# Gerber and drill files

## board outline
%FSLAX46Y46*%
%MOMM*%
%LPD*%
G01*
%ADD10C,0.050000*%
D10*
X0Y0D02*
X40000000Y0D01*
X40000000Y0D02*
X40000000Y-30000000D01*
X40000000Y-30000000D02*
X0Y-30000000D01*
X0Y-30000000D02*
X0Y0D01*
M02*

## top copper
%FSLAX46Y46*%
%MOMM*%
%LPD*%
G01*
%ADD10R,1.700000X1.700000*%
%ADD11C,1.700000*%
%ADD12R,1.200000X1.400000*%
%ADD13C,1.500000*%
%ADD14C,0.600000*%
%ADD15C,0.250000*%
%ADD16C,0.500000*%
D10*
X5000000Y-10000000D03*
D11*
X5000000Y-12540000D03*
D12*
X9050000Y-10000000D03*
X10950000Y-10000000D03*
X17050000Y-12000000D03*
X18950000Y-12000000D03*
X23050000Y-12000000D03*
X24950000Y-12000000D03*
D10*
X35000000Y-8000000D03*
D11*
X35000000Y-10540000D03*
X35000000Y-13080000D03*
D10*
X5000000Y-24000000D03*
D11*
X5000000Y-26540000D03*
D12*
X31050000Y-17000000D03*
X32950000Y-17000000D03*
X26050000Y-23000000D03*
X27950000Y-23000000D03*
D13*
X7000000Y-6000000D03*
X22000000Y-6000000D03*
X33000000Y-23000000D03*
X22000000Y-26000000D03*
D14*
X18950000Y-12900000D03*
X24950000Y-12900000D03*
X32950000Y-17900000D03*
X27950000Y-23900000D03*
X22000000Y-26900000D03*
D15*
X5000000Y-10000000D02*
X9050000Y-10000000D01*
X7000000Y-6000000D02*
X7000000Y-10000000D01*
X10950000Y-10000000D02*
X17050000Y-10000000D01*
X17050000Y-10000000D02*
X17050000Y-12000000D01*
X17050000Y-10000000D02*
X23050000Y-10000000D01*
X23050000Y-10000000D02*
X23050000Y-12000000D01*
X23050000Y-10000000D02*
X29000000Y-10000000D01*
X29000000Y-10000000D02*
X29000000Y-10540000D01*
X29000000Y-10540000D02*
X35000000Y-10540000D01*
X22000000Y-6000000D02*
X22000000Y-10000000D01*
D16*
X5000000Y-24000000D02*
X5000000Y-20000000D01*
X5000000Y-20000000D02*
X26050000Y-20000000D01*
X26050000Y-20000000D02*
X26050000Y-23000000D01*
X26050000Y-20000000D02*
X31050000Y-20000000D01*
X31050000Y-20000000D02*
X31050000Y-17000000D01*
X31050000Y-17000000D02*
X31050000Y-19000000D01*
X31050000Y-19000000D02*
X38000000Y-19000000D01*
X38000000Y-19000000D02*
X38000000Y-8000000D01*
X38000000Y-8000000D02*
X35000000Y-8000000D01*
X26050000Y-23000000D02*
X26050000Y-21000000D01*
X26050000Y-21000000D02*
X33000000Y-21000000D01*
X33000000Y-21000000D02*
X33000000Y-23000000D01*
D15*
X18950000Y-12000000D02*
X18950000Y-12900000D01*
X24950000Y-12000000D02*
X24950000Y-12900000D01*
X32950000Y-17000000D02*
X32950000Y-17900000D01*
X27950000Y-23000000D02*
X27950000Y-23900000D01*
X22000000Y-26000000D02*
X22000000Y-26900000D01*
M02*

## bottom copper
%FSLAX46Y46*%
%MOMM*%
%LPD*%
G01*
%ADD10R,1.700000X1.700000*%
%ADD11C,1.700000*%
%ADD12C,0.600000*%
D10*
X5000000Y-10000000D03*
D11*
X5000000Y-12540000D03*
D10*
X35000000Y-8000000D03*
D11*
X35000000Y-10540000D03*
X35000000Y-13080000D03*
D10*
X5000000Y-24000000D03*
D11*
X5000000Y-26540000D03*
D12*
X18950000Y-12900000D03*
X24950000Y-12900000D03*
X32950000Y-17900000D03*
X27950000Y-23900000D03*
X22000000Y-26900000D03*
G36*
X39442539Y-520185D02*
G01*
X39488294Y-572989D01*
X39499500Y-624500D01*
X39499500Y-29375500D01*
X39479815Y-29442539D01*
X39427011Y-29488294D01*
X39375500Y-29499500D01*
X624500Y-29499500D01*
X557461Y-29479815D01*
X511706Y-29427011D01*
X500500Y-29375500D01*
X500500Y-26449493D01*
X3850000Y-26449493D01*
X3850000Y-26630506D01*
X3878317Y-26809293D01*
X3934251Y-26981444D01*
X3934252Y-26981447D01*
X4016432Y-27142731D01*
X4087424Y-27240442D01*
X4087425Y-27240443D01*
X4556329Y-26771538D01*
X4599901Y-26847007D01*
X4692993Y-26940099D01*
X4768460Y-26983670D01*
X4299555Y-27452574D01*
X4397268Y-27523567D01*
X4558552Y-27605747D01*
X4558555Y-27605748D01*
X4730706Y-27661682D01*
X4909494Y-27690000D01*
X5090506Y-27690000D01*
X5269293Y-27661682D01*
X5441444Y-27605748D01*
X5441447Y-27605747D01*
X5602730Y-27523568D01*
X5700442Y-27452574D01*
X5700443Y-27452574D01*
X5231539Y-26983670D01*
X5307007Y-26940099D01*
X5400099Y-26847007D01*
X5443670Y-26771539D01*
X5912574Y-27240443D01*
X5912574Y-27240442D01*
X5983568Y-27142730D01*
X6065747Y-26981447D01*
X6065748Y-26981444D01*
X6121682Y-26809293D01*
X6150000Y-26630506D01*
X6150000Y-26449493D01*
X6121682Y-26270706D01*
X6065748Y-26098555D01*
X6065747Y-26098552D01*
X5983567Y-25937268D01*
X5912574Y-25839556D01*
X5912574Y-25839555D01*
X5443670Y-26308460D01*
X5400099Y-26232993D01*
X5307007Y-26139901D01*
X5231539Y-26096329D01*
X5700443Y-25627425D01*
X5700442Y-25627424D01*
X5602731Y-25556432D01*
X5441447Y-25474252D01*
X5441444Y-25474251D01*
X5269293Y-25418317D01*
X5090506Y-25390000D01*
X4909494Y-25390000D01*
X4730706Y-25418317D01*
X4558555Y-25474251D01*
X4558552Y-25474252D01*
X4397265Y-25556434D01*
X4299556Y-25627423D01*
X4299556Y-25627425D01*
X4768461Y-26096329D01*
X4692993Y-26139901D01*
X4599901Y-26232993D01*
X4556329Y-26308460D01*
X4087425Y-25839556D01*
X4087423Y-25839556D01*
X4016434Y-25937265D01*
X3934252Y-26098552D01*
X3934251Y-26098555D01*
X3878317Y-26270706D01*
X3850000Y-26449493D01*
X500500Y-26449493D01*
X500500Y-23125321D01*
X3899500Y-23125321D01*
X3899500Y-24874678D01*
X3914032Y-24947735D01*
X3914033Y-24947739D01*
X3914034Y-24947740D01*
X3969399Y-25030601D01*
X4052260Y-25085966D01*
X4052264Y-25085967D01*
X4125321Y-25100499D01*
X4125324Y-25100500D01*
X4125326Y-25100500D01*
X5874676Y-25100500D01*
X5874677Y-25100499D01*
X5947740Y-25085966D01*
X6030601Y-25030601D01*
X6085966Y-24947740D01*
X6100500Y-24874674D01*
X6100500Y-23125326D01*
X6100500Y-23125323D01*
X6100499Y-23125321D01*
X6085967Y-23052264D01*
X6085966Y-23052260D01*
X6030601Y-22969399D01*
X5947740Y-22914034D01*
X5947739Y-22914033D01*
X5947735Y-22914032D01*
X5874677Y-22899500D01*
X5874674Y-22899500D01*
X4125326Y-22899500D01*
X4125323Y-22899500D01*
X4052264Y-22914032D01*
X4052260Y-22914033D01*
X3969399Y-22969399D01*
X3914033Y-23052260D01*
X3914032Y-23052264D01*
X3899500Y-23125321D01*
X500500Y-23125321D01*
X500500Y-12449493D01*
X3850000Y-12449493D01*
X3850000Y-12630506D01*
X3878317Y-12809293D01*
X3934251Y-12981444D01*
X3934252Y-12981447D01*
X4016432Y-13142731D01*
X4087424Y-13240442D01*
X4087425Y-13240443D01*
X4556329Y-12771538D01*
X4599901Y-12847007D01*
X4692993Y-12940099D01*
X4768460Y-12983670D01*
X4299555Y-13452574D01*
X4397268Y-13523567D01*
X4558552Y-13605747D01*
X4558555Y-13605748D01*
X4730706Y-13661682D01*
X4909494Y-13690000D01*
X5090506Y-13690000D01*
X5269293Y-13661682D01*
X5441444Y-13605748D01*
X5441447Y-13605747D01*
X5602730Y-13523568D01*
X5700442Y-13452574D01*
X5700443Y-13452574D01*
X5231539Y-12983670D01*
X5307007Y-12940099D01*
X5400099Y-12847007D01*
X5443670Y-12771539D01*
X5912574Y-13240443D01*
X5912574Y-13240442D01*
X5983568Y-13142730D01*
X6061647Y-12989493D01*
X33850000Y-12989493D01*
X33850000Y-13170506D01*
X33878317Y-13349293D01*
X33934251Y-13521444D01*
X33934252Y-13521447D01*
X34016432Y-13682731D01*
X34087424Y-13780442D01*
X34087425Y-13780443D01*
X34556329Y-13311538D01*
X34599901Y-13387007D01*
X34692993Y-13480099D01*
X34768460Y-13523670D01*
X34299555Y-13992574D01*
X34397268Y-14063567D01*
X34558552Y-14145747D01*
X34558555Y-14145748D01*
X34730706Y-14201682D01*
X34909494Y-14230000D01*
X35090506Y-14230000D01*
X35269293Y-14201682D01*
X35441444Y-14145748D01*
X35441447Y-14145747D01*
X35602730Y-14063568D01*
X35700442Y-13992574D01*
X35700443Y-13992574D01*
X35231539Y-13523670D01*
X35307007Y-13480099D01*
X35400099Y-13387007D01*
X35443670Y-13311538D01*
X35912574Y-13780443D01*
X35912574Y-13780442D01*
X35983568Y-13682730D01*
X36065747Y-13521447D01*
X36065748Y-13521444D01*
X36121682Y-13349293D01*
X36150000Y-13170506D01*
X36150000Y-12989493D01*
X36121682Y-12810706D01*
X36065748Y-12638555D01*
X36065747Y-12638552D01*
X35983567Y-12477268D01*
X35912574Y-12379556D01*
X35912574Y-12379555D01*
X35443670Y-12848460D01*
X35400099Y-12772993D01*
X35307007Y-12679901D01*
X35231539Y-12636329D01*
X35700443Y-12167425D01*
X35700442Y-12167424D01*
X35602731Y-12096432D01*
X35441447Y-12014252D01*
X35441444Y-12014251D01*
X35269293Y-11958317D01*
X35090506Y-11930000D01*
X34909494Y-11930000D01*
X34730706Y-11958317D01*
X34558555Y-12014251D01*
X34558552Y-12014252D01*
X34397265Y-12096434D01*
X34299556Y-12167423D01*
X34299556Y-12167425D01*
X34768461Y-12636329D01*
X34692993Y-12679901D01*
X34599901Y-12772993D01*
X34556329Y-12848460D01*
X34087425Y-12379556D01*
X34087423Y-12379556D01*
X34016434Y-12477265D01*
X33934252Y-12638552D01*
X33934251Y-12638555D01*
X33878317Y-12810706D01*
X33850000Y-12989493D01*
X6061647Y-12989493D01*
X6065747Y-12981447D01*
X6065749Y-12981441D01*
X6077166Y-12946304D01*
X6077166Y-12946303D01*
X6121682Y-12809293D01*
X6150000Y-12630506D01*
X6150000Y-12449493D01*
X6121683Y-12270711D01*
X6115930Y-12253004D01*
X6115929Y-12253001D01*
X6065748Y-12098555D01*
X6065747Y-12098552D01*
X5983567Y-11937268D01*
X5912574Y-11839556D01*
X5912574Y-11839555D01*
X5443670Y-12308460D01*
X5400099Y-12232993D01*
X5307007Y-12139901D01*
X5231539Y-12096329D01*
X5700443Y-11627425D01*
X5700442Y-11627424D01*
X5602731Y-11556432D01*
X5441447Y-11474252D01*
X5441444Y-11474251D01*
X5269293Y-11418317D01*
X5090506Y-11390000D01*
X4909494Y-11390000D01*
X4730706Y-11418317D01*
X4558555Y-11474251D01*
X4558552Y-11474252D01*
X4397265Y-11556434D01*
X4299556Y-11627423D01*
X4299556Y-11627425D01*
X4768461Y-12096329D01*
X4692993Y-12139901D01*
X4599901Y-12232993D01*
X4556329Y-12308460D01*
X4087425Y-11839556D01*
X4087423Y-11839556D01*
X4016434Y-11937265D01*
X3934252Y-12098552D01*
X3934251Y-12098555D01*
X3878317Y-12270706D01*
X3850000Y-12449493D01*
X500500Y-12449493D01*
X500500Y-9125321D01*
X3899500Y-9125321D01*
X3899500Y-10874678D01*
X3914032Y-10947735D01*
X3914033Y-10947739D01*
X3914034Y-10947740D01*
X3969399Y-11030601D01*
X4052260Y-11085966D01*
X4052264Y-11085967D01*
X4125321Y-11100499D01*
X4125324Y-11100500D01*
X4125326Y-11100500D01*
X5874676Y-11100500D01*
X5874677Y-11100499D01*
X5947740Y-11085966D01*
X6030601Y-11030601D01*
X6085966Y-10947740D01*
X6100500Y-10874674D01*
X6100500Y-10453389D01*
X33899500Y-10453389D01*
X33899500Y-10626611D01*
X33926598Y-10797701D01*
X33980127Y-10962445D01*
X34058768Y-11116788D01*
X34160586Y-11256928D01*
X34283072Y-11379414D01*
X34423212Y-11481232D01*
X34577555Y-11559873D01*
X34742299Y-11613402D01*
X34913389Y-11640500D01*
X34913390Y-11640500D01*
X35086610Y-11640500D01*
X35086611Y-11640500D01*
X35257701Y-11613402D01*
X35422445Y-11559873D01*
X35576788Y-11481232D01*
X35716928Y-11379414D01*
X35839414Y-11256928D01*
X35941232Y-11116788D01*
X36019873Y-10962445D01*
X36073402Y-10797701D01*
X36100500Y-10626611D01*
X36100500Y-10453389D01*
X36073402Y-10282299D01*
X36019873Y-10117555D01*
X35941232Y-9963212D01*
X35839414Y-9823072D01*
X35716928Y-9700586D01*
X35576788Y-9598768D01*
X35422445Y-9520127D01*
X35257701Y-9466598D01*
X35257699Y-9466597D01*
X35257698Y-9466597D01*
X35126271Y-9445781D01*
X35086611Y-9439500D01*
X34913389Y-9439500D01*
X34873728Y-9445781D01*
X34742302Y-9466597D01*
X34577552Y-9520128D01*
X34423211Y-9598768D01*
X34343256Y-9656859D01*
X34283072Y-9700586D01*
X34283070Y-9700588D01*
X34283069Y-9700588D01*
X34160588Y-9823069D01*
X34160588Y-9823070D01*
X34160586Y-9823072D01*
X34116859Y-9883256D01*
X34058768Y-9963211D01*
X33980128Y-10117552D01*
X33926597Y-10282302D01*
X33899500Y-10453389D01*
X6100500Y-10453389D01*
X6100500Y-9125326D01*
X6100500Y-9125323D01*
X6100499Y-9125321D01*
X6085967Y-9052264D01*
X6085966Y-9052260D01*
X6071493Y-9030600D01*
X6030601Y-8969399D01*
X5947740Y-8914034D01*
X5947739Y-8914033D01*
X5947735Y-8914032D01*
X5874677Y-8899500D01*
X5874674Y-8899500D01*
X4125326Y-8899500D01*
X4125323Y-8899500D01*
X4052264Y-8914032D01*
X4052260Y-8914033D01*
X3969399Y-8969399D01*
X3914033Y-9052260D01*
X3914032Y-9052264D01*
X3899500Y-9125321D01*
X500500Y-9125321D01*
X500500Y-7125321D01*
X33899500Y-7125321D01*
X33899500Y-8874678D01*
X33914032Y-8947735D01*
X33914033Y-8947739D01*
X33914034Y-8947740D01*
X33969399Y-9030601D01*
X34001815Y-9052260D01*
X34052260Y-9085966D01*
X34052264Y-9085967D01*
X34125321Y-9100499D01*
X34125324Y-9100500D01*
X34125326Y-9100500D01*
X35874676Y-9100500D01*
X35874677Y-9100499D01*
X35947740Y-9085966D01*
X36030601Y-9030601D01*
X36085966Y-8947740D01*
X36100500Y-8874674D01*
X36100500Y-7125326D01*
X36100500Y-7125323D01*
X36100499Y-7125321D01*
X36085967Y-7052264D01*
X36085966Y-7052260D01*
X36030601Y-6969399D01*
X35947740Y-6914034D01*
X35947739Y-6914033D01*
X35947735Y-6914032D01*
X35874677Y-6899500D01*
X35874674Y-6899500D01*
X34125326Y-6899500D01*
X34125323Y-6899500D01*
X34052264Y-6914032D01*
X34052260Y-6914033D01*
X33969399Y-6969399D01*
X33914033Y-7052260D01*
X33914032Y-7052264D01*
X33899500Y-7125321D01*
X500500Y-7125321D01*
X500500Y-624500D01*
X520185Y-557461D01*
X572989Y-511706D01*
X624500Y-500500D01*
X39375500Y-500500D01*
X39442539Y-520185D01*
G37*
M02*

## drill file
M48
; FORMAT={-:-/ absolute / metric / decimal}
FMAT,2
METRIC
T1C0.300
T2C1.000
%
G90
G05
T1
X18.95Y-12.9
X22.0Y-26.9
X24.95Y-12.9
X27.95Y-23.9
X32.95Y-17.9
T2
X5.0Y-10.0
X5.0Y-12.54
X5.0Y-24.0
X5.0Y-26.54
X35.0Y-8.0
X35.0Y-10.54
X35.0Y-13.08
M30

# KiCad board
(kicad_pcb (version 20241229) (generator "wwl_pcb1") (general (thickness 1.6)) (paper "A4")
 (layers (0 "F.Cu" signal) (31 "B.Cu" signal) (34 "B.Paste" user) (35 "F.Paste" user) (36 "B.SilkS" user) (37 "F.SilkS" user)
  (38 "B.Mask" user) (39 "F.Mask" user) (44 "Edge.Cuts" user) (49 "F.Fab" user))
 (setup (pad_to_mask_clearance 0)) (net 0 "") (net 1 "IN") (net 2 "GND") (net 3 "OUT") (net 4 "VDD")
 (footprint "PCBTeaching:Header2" (layer "F.Cu") (at 5 10)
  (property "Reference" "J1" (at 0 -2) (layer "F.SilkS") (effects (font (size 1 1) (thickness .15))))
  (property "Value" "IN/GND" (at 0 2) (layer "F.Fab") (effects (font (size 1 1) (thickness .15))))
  (pad "1" thru_hole rect (at 0 0.0) (size 1.7 1.7) (drill 1) (layers "*.Cu" "*.Mask") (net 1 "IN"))
  (pad "2" thru_hole circle (at 0 2.54) (size 1.7 1.7) (drill 1) (layers "*.Cu" "*.Mask") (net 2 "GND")))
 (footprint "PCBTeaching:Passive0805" (layer "F.Cu") (at 10 10)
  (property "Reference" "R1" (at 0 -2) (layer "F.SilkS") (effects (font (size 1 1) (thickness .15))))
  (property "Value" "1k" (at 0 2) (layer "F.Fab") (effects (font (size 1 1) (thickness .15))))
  (pad "1" smd rect (at -0.95 0) (size 1.2 1.4) (layers "F.Cu" "F.Paste" "F.Mask") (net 1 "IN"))
  (pad "2" smd rect (at 0.95 0) (size 1.2 1.4) (layers "F.Cu" "F.Paste" "F.Mask") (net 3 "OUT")))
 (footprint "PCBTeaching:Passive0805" (layer "F.Cu") (at 18 12)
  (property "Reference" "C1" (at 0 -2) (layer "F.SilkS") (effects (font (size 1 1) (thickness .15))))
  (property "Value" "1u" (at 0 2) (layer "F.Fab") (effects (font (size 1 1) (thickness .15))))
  (pad "1" smd rect (at -0.95 0) (size 1.2 1.4) (layers "F.Cu" "F.Paste" "F.Mask") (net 3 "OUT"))
  (pad "2" smd rect (at 0.95 0) (size 1.2 1.4) (layers "F.Cu" "F.Paste" "F.Mask") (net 2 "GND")))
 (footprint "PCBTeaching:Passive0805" (layer "F.Cu") (at 24 12)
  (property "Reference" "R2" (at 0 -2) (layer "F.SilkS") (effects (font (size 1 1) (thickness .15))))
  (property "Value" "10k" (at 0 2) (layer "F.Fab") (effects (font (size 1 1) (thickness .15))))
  (pad "1" smd rect (at -0.95 0) (size 1.2 1.4) (layers "F.Cu" "F.Paste" "F.Mask") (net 3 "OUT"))
  (pad "2" smd rect (at 0.95 0) (size 1.2 1.4) (layers "F.Cu" "F.Paste" "F.Mask") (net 2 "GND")))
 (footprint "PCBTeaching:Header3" (layer "F.Cu") (at 35 8)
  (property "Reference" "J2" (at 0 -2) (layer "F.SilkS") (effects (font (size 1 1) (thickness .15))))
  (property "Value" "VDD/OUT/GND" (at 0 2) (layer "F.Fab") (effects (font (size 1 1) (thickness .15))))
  (pad "1" thru_hole rect (at 0 0.0) (size 1.7 1.7) (drill 1) (layers "*.Cu" "*.Mask") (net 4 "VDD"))
  (pad "2" thru_hole circle (at 0 2.54) (size 1.7 1.7) (drill 1) (layers "*.Cu" "*.Mask") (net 3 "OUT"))
  (pad "3" thru_hole circle (at 0 5.08) (size 1.7 1.7) (drill 1) (layers "*.Cu" "*.Mask") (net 2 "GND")))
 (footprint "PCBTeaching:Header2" (layer "F.Cu") (at 5 24)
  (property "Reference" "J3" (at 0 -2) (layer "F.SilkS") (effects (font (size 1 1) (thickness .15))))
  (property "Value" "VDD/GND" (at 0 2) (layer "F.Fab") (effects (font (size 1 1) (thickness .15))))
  (pad "1" thru_hole rect (at 0 0.0) (size 1.7 1.7) (drill 1) (layers "*.Cu" "*.Mask") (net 4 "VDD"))
  (pad "2" thru_hole circle (at 0 2.54) (size 1.7 1.7) (drill 1) (layers "*.Cu" "*.Mask") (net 2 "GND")))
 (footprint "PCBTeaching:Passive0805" (layer "F.Cu") (at 32 17)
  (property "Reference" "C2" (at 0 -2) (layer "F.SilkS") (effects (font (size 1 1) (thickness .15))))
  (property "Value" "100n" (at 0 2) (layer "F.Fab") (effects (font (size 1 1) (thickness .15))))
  (pad "1" smd rect (at -0.95 0) (size 1.2 1.4) (layers "F.Cu" "F.Paste" "F.Mask") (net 4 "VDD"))
  (pad "2" smd rect (at 0.95 0) (size 1.2 1.4) (layers "F.Cu" "F.Paste" "F.Mask") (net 2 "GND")))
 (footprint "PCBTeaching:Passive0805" (layer "F.Cu") (at 27 23)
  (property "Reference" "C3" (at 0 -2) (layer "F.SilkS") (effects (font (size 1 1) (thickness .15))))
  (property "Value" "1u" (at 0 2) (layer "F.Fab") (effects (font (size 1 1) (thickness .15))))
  (pad "1" smd rect (at -0.95 0) (size 1.2 1.4) (layers "F.Cu" "F.Paste" "F.Mask") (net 4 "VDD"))
  (pad "2" smd rect (at 0.95 0) (size 1.2 1.4) (layers "F.Cu" "F.Paste" "F.Mask") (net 2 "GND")))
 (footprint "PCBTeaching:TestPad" (layer "F.Cu") (at 7 6)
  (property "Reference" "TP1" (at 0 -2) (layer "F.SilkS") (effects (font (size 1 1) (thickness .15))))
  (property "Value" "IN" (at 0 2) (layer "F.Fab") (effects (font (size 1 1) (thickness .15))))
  (pad "1" smd circle (at 0 0.0) (size 1.5 1.5) (layers "F.Cu" "F.Paste" "F.Mask") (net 1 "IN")))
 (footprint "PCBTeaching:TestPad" (layer "F.Cu") (at 22 6)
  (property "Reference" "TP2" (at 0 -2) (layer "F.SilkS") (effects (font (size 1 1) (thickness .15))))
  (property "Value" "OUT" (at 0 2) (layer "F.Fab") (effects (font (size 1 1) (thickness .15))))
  (pad "1" smd circle (at 0 0.0) (size 1.5 1.5) (layers "F.Cu" "F.Paste" "F.Mask") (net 3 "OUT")))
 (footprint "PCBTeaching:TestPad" (layer "F.Cu") (at 33 23)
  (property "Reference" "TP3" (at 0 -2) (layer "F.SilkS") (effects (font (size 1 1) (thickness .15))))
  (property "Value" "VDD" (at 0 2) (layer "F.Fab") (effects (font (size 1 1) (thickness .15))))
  (pad "1" smd circle (at 0 0.0) (size 1.5 1.5) (layers "F.Cu" "F.Paste" "F.Mask") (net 4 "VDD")))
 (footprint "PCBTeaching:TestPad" (layer "F.Cu") (at 22 26)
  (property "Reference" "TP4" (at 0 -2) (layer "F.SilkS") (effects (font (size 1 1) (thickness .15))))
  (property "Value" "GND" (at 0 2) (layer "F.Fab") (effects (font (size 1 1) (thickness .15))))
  (pad "1" smd circle (at 0 0.0) (size 1.5 1.5) (layers "F.Cu" "F.Paste" "F.Mask") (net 2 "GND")))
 (segment (start 5 10) (end 9.05 10) (width .25) (layer "F.Cu") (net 1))
 (segment (start 7 6) (end 7 10) (width .25) (layer "F.Cu") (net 1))
 (segment (start 10.95 10) (end 17.05 10) (width .25) (layer "F.Cu") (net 3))
 (segment (start 17.05 10) (end 17.05 12) (width .25) (layer "F.Cu") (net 3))
 (segment (start 17.05 10) (end 23.05 10) (width .25) (layer "F.Cu") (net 3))
 (segment (start 23.05 10) (end 23.05 12) (width .25) (layer "F.Cu") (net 3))
 (segment (start 23.05 10) (end 29 10) (width .25) (layer "F.Cu") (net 3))
 (segment (start 29 10) (end 29 10.54) (width .25) (layer "F.Cu") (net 3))
 (segment (start 29 10.54) (end 35 10.54) (width .25) (layer "F.Cu") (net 3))
 (segment (start 22 6) (end 22 10) (width .25) (layer "F.Cu") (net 3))
 (segment (start 5 24) (end 5 20) (width .5) (layer "F.Cu") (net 4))
 (segment (start 5 20) (end 26.05 20) (width .5) (layer "F.Cu") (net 4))
 (segment (start 26.05 20) (end 26.05 23) (width .5) (layer "F.Cu") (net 4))
 (segment (start 26.05 20) (end 31.05 20) (width .5) (layer "F.Cu") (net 4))
 (segment (start 31.05 20) (end 31.05 17) (width .5) (layer "F.Cu") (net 4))
 (segment (start 31.05 17) (end 31.05 19) (width .5) (layer "F.Cu") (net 4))
 (segment (start 31.05 19) (end 38 19) (width .5) (layer "F.Cu") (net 4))
 (segment (start 38 19) (end 38 8) (width .5) (layer "F.Cu") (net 4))
 (segment (start 38 8) (end 35 8) (width .5) (layer "F.Cu") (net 4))
 (segment (start 26.05 23) (end 26.05 21) (width .5) (layer "F.Cu") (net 4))
 (segment (start 26.05 21) (end 33 21) (width .5) (layer "F.Cu") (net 4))
 (segment (start 33 21) (end 33 23) (width .5) (layer "F.Cu") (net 4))
 (segment (start 18.95 12) (end 18.95 12.9) (width .25) (layer "F.Cu") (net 2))
 (segment (start 24.95 12) (end 24.95 12.9) (width .25) (layer "F.Cu") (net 2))
 (segment (start 32.95 17) (end 32.95 17.9) (width .25) (layer "F.Cu") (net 2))
 (segment (start 27.95 23) (end 27.95 23.9) (width .25) (layer "F.Cu") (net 2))
 (segment (start 22 26.0) (end 22 26.9) (width .25) (layer "F.Cu") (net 2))
 (via (at 18.95 12.9) (size .6) (drill .3) (layers "F.Cu" "B.Cu") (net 2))
 (via (at 24.95 12.9) (size .6) (drill .3) (layers "F.Cu" "B.Cu") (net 2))
 (via (at 32.95 17.9) (size .6) (drill .3) (layers "F.Cu" "B.Cu") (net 2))
 (via (at 27.95 23.9) (size .6) (drill .3) (layers "F.Cu" "B.Cu") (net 2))
 (via (at 22 26.9) (size .6) (drill .3) (layers "F.Cu" "B.Cu") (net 2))
 (gr_line (start 0 0) (end 40 0) (stroke (width .05) (type default)) (layer "Edge.Cuts"))
 (gr_line (start 40 0) (end 40 30) (stroke (width .05) (type default)) (layer "Edge.Cuts"))
 (gr_line (start 40 30) (end 0 30) (stroke (width .05) (type default)) (layer "Edge.Cuts"))
 (gr_line (start 0 30) (end 0 0) (stroke (width .05) (type default)) (layer "Edge.Cuts"))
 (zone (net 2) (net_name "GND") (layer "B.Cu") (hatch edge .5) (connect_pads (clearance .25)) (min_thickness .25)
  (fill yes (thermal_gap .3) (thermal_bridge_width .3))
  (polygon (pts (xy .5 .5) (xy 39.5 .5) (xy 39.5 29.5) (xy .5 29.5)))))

